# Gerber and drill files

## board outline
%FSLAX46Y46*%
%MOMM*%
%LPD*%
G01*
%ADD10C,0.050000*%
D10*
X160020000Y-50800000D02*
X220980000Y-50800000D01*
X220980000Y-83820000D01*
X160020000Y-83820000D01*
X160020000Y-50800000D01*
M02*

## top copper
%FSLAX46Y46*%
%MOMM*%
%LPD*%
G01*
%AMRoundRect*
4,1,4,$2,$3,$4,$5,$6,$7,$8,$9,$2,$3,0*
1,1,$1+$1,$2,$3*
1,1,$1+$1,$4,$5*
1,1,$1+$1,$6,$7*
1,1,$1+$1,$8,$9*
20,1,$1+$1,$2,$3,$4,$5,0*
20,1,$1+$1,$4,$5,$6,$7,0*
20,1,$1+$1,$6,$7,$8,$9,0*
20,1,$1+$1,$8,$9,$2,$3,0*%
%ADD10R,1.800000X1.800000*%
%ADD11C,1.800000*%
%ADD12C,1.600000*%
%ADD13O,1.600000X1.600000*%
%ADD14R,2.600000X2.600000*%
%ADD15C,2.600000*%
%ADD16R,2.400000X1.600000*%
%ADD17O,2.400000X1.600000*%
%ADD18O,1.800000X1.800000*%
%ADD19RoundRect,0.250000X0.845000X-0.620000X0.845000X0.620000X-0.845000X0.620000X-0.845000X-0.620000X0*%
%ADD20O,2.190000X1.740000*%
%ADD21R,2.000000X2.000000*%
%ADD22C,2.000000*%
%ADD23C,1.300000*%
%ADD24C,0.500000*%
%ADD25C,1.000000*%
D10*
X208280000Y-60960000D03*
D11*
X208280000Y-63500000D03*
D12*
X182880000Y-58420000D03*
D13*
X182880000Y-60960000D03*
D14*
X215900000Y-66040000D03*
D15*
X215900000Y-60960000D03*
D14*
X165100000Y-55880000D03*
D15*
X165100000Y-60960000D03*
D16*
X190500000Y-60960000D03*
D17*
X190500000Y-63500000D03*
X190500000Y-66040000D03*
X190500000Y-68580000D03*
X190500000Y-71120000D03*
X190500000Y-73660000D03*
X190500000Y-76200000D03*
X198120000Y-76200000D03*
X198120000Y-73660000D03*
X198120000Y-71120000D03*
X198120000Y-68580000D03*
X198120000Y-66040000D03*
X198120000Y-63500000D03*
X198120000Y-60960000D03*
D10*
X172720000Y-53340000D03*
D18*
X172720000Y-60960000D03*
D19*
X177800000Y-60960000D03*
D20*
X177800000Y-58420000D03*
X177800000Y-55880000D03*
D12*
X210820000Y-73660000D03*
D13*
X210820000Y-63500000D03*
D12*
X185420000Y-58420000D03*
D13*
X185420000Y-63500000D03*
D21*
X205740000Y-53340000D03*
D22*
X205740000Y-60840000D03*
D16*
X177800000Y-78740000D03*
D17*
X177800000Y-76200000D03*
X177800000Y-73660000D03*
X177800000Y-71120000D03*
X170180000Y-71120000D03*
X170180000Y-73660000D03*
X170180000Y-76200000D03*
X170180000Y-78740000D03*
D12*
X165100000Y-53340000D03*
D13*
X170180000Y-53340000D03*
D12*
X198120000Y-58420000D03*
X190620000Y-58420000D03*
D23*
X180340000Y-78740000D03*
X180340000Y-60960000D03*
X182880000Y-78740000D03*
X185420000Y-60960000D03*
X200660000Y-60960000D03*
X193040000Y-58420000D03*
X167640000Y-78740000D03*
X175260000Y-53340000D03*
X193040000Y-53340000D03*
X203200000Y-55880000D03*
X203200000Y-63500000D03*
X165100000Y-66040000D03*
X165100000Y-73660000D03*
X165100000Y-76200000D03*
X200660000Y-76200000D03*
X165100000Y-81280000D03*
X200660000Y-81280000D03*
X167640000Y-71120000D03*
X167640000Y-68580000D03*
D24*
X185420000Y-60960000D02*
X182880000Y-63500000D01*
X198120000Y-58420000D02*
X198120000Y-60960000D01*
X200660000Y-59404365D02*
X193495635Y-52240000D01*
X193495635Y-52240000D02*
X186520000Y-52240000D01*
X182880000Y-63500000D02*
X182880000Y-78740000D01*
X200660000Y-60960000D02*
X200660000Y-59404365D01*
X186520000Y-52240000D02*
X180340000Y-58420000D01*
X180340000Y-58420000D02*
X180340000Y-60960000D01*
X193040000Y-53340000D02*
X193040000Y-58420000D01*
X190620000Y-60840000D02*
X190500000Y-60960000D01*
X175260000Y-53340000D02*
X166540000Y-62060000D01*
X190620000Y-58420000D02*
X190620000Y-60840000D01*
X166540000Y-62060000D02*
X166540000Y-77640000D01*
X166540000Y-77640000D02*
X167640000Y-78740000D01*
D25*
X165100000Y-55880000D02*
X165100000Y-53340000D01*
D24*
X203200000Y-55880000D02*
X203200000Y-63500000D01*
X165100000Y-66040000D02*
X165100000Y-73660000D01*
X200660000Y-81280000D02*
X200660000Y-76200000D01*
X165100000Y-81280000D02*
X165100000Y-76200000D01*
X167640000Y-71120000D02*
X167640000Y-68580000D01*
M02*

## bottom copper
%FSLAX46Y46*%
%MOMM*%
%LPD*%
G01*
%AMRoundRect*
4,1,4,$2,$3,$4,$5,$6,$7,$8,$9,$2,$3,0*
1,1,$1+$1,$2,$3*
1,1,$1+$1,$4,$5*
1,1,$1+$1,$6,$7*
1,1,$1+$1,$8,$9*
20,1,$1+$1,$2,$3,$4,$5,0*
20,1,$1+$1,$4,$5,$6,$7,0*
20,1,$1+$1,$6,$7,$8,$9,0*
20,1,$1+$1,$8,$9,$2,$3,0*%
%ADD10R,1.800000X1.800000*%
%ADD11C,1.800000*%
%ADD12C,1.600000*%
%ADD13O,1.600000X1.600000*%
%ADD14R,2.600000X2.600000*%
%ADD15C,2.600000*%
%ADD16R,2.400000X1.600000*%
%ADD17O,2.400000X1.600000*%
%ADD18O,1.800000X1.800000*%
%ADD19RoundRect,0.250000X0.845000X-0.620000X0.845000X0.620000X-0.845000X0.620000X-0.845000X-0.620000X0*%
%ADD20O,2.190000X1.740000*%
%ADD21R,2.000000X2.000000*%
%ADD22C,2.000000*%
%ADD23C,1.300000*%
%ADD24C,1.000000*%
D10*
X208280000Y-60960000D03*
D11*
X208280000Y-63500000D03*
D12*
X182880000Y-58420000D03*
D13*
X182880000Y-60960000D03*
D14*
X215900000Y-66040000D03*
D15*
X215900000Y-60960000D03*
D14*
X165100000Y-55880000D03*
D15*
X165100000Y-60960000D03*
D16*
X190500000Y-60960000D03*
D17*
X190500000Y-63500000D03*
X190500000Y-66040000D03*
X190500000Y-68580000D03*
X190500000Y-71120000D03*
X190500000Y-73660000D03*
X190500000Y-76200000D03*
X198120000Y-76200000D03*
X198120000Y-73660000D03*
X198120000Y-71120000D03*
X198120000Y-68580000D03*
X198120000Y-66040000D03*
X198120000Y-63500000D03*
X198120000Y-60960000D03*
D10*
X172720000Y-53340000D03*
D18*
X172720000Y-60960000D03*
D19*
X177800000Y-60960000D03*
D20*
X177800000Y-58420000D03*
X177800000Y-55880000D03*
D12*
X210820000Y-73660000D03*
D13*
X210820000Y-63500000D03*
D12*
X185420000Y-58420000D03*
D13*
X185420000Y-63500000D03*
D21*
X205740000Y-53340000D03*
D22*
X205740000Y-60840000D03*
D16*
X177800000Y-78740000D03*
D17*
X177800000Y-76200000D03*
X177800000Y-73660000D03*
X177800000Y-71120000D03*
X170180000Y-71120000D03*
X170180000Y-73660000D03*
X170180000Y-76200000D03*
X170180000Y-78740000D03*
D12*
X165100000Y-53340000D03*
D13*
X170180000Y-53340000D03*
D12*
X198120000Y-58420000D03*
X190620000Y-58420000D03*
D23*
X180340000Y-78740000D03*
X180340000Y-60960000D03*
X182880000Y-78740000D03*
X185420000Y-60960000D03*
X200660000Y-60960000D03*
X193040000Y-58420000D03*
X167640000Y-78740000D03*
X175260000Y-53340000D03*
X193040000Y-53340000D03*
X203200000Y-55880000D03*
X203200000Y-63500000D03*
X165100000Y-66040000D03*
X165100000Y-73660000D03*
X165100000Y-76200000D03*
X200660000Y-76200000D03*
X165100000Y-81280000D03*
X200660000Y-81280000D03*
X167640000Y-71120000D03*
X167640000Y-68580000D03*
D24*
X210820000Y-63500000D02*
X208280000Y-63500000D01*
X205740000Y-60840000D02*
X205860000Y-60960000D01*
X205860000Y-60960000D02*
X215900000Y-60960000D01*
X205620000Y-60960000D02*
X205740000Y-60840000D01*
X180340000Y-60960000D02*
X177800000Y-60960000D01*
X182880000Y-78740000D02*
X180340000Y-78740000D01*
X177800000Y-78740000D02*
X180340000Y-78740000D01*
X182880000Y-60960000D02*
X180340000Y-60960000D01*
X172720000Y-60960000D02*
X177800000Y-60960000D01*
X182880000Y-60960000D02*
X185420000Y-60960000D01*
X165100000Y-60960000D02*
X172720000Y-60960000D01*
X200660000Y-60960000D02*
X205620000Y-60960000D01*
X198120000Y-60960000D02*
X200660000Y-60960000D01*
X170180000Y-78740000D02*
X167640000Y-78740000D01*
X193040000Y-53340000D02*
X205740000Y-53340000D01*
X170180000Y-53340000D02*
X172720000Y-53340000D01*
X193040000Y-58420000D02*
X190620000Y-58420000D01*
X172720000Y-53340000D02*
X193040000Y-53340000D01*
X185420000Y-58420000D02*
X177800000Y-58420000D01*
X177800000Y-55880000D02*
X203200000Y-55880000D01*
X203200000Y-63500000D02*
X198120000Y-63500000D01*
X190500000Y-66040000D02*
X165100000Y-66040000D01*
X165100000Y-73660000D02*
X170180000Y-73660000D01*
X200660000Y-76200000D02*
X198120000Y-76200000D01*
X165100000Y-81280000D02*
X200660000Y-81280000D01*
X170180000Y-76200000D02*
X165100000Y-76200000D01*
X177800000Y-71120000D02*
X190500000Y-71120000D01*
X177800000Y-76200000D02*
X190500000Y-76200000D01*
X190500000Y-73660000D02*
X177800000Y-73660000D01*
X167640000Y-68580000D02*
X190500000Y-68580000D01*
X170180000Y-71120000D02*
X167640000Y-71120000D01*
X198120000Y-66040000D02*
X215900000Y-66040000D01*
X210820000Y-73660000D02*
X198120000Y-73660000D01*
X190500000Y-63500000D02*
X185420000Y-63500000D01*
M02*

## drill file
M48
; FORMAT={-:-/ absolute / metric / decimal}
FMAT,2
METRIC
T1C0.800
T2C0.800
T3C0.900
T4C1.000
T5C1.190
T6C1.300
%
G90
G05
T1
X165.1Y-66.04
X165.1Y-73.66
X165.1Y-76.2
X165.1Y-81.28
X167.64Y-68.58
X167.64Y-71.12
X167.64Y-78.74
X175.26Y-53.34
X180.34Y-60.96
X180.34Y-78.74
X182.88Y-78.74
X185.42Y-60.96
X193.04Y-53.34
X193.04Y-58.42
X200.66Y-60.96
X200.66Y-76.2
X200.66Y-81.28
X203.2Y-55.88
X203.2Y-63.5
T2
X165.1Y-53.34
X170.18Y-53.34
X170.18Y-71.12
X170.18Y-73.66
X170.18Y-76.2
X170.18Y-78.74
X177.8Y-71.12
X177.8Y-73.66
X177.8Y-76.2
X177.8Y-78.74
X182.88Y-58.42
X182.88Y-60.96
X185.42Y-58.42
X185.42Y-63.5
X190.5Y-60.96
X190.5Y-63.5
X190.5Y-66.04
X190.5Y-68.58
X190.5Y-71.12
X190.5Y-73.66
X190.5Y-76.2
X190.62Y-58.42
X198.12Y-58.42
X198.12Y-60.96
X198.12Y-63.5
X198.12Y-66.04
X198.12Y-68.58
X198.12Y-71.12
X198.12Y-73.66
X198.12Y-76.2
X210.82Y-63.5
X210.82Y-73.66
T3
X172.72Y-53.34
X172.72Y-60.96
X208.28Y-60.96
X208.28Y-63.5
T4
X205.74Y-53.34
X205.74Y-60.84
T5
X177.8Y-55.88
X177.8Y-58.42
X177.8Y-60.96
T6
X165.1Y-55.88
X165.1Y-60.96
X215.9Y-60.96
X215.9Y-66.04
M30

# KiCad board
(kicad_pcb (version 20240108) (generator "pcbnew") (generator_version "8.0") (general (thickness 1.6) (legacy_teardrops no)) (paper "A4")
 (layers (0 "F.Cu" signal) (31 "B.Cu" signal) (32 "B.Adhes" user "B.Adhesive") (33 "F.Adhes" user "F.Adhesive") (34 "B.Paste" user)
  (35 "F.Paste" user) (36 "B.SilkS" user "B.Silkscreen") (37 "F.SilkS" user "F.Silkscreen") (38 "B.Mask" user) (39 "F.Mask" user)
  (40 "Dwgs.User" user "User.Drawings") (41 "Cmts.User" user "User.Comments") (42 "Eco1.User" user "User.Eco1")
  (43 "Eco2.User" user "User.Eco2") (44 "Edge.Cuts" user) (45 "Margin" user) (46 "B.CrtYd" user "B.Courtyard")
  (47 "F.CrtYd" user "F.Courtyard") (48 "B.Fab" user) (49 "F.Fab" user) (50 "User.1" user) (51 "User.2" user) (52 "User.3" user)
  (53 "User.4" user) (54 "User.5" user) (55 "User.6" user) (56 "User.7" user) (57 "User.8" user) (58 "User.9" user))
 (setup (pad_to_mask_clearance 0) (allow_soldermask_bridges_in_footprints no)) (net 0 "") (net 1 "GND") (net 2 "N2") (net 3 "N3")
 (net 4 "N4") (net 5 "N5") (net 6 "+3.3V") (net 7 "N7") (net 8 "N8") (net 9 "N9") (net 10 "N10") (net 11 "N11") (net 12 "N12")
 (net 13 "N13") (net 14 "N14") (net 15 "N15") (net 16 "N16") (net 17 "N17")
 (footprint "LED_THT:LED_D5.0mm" (layer "F.Cu") (at 208.28 60.96 -90)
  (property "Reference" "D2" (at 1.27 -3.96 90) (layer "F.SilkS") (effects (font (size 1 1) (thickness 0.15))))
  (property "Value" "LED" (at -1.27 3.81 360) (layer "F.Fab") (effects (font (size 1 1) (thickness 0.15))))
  (pad "1" thru_hole rect (at 0 0 270) (size 1.8 1.8) (drill 0.9) (layers "*.Cu" "*.Mask") (remove_unused_layers no) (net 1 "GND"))
  (pad "2" thru_hole circle (at 2.54 0 270) (size 1.8 1.8) (drill 0.9) (layers "*.Cu" "*.Mask") (remove_unused_layers no) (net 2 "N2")))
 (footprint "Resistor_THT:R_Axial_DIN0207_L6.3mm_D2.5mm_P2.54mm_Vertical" (layer "F.Cu") (at 182.88 58.42 -90)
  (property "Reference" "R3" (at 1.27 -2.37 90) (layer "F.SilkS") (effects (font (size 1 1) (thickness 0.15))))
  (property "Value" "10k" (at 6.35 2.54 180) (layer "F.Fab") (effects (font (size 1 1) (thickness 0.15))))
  (pad "1" thru_hole circle (at 0 0 270) (size 1.6 1.6) (drill 0.8) (layers "*.Cu" "*.Mask") (remove_unused_layers no) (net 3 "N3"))
  (pad "2" thru_hole oval (at 2.54 0 270) (size 1.6 1.6) (drill 0.8) (layers "*.Cu" "*.Mask") (remove_unused_layers no) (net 1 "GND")))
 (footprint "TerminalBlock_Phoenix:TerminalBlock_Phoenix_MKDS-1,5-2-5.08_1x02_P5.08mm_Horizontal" (layer "F.Cu") (at 215.9 66.04 90)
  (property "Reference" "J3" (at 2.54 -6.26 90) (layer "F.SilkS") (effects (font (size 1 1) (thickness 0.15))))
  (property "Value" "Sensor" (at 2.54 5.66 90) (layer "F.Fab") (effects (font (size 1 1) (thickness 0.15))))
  (pad "1" thru_hole rect (at 0 0 90) (size 2.6 2.6) (drill 1.3) (layers "*.Cu" "*.Mask") (remove_unused_layers no) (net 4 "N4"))
  (pad "2" thru_hole circle (at 5.08 0 90) (size 2.6 2.6) (drill 1.3) (layers "*.Cu" "*.Mask") (remove_unused_layers no) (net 1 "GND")))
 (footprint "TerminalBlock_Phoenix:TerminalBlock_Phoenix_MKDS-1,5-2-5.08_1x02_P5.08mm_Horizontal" (layer "F.Cu") (at 165.1 55.88 -90)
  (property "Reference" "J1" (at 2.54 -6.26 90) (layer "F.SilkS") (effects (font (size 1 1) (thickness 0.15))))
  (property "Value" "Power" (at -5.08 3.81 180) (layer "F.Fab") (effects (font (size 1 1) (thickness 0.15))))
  (pad "1" thru_hole rect (at 0 0 270) (size 2.6 2.6) (drill 1.3) (layers "*.Cu" "*.Mask") (remove_unused_layers no) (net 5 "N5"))
  (pad "2" thru_hole circle (at 5.08 0 270) (size 2.6 2.6) (drill 1.3) (layers "*.Cu" "*.Mask") (remove_unused_layers no) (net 1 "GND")))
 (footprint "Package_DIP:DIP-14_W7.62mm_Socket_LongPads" (layer "F.Cu") (at 190.5 60.96)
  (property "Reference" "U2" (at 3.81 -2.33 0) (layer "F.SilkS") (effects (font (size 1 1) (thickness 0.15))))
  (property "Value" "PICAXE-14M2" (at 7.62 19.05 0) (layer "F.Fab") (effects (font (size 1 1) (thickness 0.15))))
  (pad "1" thru_hole rect (at 0 0) (size 2.4 1.6) (drill 0.8) (layers "*.Cu" "*.Mask") (remove_unused_layers no) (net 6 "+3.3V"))
  (pad "2" thru_hole oval (at 0 2.54) (size 2.4 1.6) (drill 0.8) (layers "*.Cu" "*.Mask") (remove_unused_layers no) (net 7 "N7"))
  (pad "3" thru_hole oval (at 0 5.08) (size 2.4 1.6) (drill 0.8) (layers "*.Cu" "*.Mask") (remove_unused_layers no) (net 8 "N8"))
  (pad "4" thru_hole oval (at 0 7.62) (size 2.4 1.6) (drill 0.8) (layers "*.Cu" "*.Mask") (remove_unused_layers no) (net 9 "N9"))
  (pad "5" thru_hole oval (at 0 10.16) (size 2.4 1.6) (drill 0.8) (layers "*.Cu" "*.Mask") (remove_unused_layers no) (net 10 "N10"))
  (pad "6" thru_hole oval (at 0 12.7) (size 2.4 1.6) (drill 0.8) (layers "*.Cu" "*.Mask") (remove_unused_layers no) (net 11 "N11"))
  (pad "7" thru_hole oval (at 0 15.24) (size 2.4 1.6) (drill 0.8) (layers "*.Cu" "*.Mask") (remove_unused_layers no) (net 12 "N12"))
  (pad "8" thru_hole oval (at 7.62 15.24) (size 2.4 1.6) (drill 0.8) (layers "*.Cu" "*.Mask") (remove_unused_layers no) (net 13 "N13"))
  (pad "9" thru_hole oval (at 7.62 12.7) (size 2.4 1.6) (drill 0.8) (layers "*.Cu" "*.Mask") (remove_unused_layers no) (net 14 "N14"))
  (pad "10" thru_hole oval (at 7.62 10.16) (size 2.4 1.6) (drill 0.8) (layers "*.Cu" "*.Mask") (remove_unused_layers no) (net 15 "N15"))
  (pad "11" thru_hole oval (at 7.62 7.62) (size 2.4 1.6) (drill 0.8) (layers "*.Cu" "*.Mask") (remove_unused_layers no) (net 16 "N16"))
  (pad "12" thru_hole oval (at 7.62 5.08) (size 2.4 1.6) (drill 0.8) (layers "*.Cu" "*.Mask") (remove_unused_layers no) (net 4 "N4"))
  (pad "13" thru_hole oval (at 7.62 2.54) (size 2.4 1.6) (drill 0.8) (layers "*.Cu" "*.Mask") (remove_unused_layers no) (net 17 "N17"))
  (pad "14" thru_hole oval (at 7.62 0) (size 2.4 1.6) (drill 0.8) (layers "*.Cu" "*.Mask") (remove_unused_layers no) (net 1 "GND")))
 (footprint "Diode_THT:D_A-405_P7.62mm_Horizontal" (layer "F.Cu") (at 172.72 53.34 -90)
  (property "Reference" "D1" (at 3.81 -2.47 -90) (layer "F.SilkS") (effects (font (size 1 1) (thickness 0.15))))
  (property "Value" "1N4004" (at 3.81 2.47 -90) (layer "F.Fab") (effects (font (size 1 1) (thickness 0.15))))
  (pad "1" thru_hole rect (at 0 0 270) (size 1.8 1.8) (drill 0.9) (layers "*.Cu" "*.Mask") (remove_unused_layers no) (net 6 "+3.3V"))
  (pad "2" thru_hole oval (at 7.62 0 270) (size 1.8 1.8) (drill 0.9) (layers "*.Cu" "*.Mask") (remove_unused_layers no) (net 1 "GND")))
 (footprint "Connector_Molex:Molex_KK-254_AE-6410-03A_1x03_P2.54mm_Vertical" (layer "F.Cu") (at 177.8 60.96 90)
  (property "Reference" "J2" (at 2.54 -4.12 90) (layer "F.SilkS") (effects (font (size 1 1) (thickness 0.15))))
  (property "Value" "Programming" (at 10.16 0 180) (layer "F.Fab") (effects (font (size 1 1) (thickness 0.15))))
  (pad "1" thru_hole roundrect (at 0 0 90) (size 1.74 2.19) (drill 1.19) (layers "*.Cu" "*.Mask") (remove_unused_layers no)
   (roundrect_rratio 0.143678) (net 1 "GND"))
  (pad "2" thru_hole oval (at 2.54 0 90) (size 1.74 2.19) (drill 1.19) (layers "*.Cu" "*.Mask") (remove_unused_layers no) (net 3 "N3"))
  (pad "3" thru_hole oval (at 5.08 0 90) (size 1.74 2.19) (drill 1.19) (layers "*.Cu" "*.Mask") (remove_unused_layers no) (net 17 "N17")))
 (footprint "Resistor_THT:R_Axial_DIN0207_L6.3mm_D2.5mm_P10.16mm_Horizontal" (layer "F.Cu") (at 210.82 73.66 90)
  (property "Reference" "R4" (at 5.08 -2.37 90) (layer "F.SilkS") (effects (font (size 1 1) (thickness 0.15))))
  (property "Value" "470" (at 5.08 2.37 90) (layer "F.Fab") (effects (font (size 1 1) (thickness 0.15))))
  (pad "1" thru_hole circle (at 0 0 90) (size 1.6 1.6) (drill 0.8) (layers "*.Cu" "*.Mask") (remove_unused_layers no) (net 14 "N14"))
  (pad "2" thru_hole oval (at 10.16 0 90) (size 1.6 1.6) (drill 0.8) (layers "*.Cu" "*.Mask") (remove_unused_layers no) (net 2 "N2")))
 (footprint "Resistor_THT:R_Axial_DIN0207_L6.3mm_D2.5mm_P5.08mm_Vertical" (layer "F.Cu") (at 185.42 58.42 -90)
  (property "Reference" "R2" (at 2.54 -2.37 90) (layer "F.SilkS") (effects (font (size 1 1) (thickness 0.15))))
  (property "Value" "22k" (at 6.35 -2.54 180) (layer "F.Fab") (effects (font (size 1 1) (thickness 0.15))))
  (pad "1" thru_hole circle (at 0 0 270) (size 1.6 1.6) (drill 0.8) (layers "*.Cu" "*.Mask") (remove_unused_layers no) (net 3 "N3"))
  (pad "2" thru_hole oval (at 5.08 0 270) (size 1.6 1.6) (drill 0.8) (layers "*.Cu" "*.Mask") (remove_unused_layers no) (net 7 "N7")))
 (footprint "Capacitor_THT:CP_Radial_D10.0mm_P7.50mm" (layer "F.Cu") (at 205.74 53.34 -90)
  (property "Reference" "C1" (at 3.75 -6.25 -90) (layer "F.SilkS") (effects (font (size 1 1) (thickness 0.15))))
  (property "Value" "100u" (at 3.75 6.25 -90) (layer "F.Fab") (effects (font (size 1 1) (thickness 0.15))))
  (pad "1" thru_hole rect (at 0 0 270) (size 2 2) (drill 1) (layers "*.Cu" "*.Mask") (remove_unused_layers no) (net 6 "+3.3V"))
  (pad "2" thru_hole circle (at 7.5 0 270) (size 2 2) (drill 1) (layers "*.Cu" "*.Mask") (remove_unused_layers no) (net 1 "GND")))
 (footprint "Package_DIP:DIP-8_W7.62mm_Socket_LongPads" (layer "F.Cu") (at 177.8 78.74 180)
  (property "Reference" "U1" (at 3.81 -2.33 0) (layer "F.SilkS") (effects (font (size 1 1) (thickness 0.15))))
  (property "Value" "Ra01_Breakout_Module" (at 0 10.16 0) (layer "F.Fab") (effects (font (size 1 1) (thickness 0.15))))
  (pad "1" thru_hole rect (at 0 0 180) (size 2.4 1.6) (drill 0.8) (layers "*.Cu" "*.Mask") (remove_unused_layers no) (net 1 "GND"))
  (pad "2" thru_hole oval (at 0 2.54 180) (size 2.4 1.6) (drill 0.8) (layers "*.Cu" "*.Mask") (remove_unused_layers no) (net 12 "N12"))
  (pad "3" thru_hole oval (at 0 5.08 180) (size 2.4 1.6) (drill 0.8) (layers "*.Cu" "*.Mask") (remove_unused_layers no) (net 11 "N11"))
  (pad "4" thru_hole oval (at 0 7.62 180) (size 2.4 1.6) (drill 0.8) (layers "*.Cu" "*.Mask") (remove_unused_layers no) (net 10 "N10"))
  (pad "5" thru_hole oval (at 7.62 7.62 180) (size 2.4 1.6) (drill 0.8) (layers "*.Cu" "*.Mask") (remove_unused_layers no) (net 9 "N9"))
  (pad "6" thru_hole oval (at 7.62 5.08 180) (size 2.4 1.6) (drill 0.8) (layers "*.Cu" "*.Mask") (remove_unused_layers no) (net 8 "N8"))
  (pad "7" thru_hole oval (at 7.62 2.54 180) (size 2.4 1.6) (drill 0.8) (layers "*.Cu" "*.Mask") (remove_unused_layers no) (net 13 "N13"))
  (pad "8" thru_hole oval (at 7.62 0 180) (size 2.4 1.6) (drill 0.8) (layers "*.Cu" "*.Mask") (remove_unused_layers no) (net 6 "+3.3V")))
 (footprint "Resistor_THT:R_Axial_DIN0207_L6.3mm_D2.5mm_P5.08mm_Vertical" (layer "F.Cu") (at 165.1 53.34)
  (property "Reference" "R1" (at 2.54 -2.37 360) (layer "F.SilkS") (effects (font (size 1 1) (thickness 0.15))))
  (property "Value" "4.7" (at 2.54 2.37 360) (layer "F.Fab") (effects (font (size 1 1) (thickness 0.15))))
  (pad "1" thru_hole circle (at 0 0) (size 1.6 1.6) (drill 0.8) (layers "*.Cu" "*.Mask") (remove_unused_layers no) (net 5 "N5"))
  (pad "2" thru_hole oval (at 5.08 0) (size 1.6 1.6) (drill 0.8) (layers "*.Cu" "*.Mask") (remove_unused_layers no) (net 6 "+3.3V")))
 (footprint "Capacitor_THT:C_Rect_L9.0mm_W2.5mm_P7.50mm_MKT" (layer "F.Cu") (at 198.12 58.42 180)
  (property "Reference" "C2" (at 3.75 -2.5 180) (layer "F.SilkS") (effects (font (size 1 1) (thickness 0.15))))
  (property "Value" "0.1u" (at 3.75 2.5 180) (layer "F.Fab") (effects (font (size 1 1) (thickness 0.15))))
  (pad "1" thru_hole circle (at 0 0 180) (size 1.6 1.6) (drill 0.8) (layers "*.Cu" "*.Mask") (remove_unused_layers no) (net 1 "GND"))
  (pad "2" thru_hole circle (at 7.5 0 180) (size 1.6 1.6) (drill 0.8) (layers "*.Cu" "*.Mask") (remove_unused_layers no) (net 6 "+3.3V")))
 (gr_rect (start 160.02 50.8) (end 220.98 83.82) (stroke (width 0.05) (type default)) (fill none) (layer "Edge.Cuts"))
 (segment (start 210.82 63.5) (end 208.28 63.5) (width 1) (layer "B.Cu") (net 2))
 (segment (start 185.42 60.96) (end 182.88 63.5) (width 0.5) (layer "F.Cu") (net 1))
 (segment (start 198.12 58.42) (end 198.12 60.96) (width 0.5) (layer "F.Cu") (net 1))
 (segment (start 200.66 59.404365) (end 193.495635 52.24) (width 0.5) (layer "F.Cu") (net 1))
 (segment (start 193.495635 52.24) (end 186.52 52.24) (width 0.5) (layer "F.Cu") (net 1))
 (segment (start 182.88 63.5) (end 182.88 78.74) (width 0.5) (layer "F.Cu") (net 1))
 (segment (start 200.66 60.96) (end 200.66 59.404365) (width 0.5) (layer "F.Cu") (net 1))
 (segment (start 186.52 52.24) (end 180.34 58.42) (width 0.5) (layer "F.Cu") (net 1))
 (segment (start 180.34 58.42) (end 180.34 60.96) (width 0.5) (layer "F.Cu") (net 1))
 (via (at 180.34 78.74) (size 1.3) (drill 0.8) (layers "F.Cu" "B.Cu") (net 1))
 (via (at 180.34 60.96) (size 1.3) (drill 0.8) (layers "F.Cu" "B.Cu") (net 1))
 (via (at 182.88 78.74) (size 1.3) (drill 0.8) (layers "F.Cu" "B.Cu") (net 1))
 (via (at 185.42 60.96) (size 1.3) (drill 0.8) (layers "F.Cu" "B.Cu") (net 1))
 (via (at 200.66 60.96) (size 1.3) (drill 0.8) (layers "F.Cu" "B.Cu") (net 1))
 (segment (start 205.74 60.84) (end 205.86 60.96) (width 1) (layer "B.Cu") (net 1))
 (segment (start 205.86 60.96) (end 215.9 60.96) (width 1) (layer "B.Cu") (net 1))
 (segment (start 205.62 60.96) (end 205.74 60.84) (width 1) (layer "B.Cu") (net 1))
 (segment (start 180.34 60.96) (end 177.8 60.96) (width 1) (layer "B.Cu") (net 1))
 (segment (start 182.88 78.74) (end 180.34 78.74) (width 1) (layer "B.Cu") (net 1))
 (segment (start 177.8 78.74) (end 180.34 78.74) (width 1) (layer "B.Cu") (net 1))
 (segment (start 182.88 60.96) (end 180.34 60.96) (width 1) (layer "B.Cu") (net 1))
 (segment (start 172.72 60.96) (end 177.8 60.96) (width 1) (layer "B.Cu") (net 1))
 (segment (start 182.88 60.96) (end 185.42 60.96) (width 1) (layer "B.Cu") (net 1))
 (segment (start 165.1 60.96) (end 172.72 60.96) (width 1) (layer "B.Cu") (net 1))
 (segment (start 200.66 60.96) (end 205.62 60.96) (width 1) (layer "B.Cu") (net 1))
 (segment (start 198.12 60.96) (end 200.66 60.96) (width 1) (layer "B.Cu") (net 1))
 (segment (start 193.04 53.34) (end 193.04 58.42) (width 0.5) (layer "F.Cu") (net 6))
 (segment (start 190.62 60.84) (end 190.5 60.96) (width 0.5) (layer "F.Cu") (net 6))
 (segment (start 175.26 53.34) (end 166.54 62.06) (width 0.5) (layer "F.Cu") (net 6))
 (segment (start 190.62 58.42) (end 190.62 60.84) (width 0.5) (layer "F.Cu") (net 6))
 (segment (start 166.54 62.06) (end 166.54 77.64) (width 0.5) (layer "F.Cu") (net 6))
 (segment (start 166.54 77.64) (end 167.64 78.74) (width 0.5) (layer "F.Cu") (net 6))
 (via (at 193.04 58.42) (size 1.3) (drill 0.8) (layers "F.Cu" "B.Cu") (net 6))
 (via (at 167.64 78.74) (size 1.3) (drill 0.8) (layers "F.Cu" "B.Cu") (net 6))
 (via (at 175.26 53.34) (size 1.3) (drill 0.8) (layers "F.Cu" "B.Cu") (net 6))
 (via (at 193.04 53.34) (size 1.3) (drill 0.8) (layers "F.Cu" "B.Cu") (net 6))
 (segment (start 170.18 78.74) (end 167.64 78.74) (width 1) (layer "B.Cu") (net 6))
 (segment (start 193.04 53.34) (end 205.74 53.34) (width 1) (layer "B.Cu") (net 6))
 (segment (start 170.18 53.34) (end 172.72 53.34) (width 1) (layer "B.Cu") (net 6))
 (segment (start 193.04 58.42) (end 190.62 58.42) (width 1) (layer "B.Cu") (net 6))
 (segment (start 172.72 53.34) (end 193.04 53.34) (width 1) (layer "B.Cu") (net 6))
 (segment (start 165.1 55.88) (end 165.1 53.34) (width 1) (layer "F.Cu") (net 5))
 (segment (start 185.42 58.42) (end 177.8 58.42) (width 1) (layer "B.Cu") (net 3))
 (segment (start 203.2 55.88) (end 203.2 63.5) (width 0.5) (layer "F.Cu") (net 17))
 (via (at 203.2 55.88) (size 1.3) (drill 0.8) (layers "F.Cu" "B.Cu") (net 17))
 (via (at 203.2 63.5) (size 1.3) (drill 0.8) (layers "F.Cu" "B.Cu") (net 17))
 (segment (start 177.8 55.88) (end 203.2 55.88) (width 1) (layer "B.Cu") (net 17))
 (segment (start 203.2 63.5) (end 198.12 63.5) (width 1) (layer "B.Cu") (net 17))
 (segment (start 165.1 66.04) (end 165.1 73.66) (width 0.5) (layer "F.Cu") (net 8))
 (via (at 165.1 66.04) (size 1.3) (drill 0.8) (layers "F.Cu" "B.Cu") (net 8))
 (via (at 165.1 73.66) (size 1.3) (drill 0.8) (layers "F.Cu" "B.Cu") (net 8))
 (segment (start 190.5 66.04) (end 165.1 66.04) (width 1) (layer "B.Cu") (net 8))
 (segment (start 165.1 73.66) (end 170.18 73.66) (width 1) (layer "B.Cu") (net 8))
 (segment (start 200.66 81.28) (end 200.66 76.2) (width 0.5) (layer "F.Cu") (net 13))
 (segment (start 165.1 81.28) (end 165.1 76.2) (width 0.5) (layer "F.Cu") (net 13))
 (via (at 165.1 76.2) (size 1.3) (drill 0.8) (layers "F.Cu" "B.Cu") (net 13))
 (via (at 200.66 76.2) (size 1.3) (drill 0.8) (layers "F.Cu" "B.Cu") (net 13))
 (via (at 165.1 81.28) (size 1.3) (drill 0.8) (layers "F.Cu" "B.Cu") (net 13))
 (via (at 200.66 81.28) (size 1.3) (drill 0.8) (layers "F.Cu" "B.Cu") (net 13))
 (segment (start 200.66 76.2) (end 198.12 76.2) (width 1) (layer "B.Cu") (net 13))
 (segment (start 165.1 81.28) (end 200.66 81.28) (width 1) (layer "B.Cu") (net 13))
 (segment (start 170.18 76.2) (end 165.1 76.2) (width 1) (layer "B.Cu") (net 13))
 (segment (start 177.8 71.12) (end 190.5 71.12) (width 1) (layer "B.Cu") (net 10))
 (segment (start 177.8 76.2) (end 190.5 76.2) (width 1) (layer "B.Cu") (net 12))
 (segment (start 190.5 73.66) (end 177.8 73.66) (width 1) (layer "B.Cu") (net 11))
 (segment (start 167.64 71.12) (end 167.64 68.58) (width 0.5) (layer "F.Cu") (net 9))
 (via (at 167.64 71.12) (size 1.3) (drill 0.8) (layers "F.Cu" "B.Cu") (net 9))
 (via (at 167.64 68.58) (size 1.3) (drill 0.8) (layers "F.Cu" "B.Cu") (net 9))
 (segment (start 167.64 68.58) (end 190.5 68.58) (width 1) (layer "B.Cu") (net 9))
 (segment (start 170.18 71.12) (end 167.64 71.12) (width 1) (layer "B.Cu") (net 9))
 (segment (start 198.12 66.04) (end 215.9 66.04) (width 1) (layer "B.Cu") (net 4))
 (segment (start 210.82 73.66) (end 198.12 73.66) (width 1) (layer "B.Cu") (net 14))
 (segment (start 190.5 63.5) (end 185.42 63.5) (width 1) (layer "B.Cu") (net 7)))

